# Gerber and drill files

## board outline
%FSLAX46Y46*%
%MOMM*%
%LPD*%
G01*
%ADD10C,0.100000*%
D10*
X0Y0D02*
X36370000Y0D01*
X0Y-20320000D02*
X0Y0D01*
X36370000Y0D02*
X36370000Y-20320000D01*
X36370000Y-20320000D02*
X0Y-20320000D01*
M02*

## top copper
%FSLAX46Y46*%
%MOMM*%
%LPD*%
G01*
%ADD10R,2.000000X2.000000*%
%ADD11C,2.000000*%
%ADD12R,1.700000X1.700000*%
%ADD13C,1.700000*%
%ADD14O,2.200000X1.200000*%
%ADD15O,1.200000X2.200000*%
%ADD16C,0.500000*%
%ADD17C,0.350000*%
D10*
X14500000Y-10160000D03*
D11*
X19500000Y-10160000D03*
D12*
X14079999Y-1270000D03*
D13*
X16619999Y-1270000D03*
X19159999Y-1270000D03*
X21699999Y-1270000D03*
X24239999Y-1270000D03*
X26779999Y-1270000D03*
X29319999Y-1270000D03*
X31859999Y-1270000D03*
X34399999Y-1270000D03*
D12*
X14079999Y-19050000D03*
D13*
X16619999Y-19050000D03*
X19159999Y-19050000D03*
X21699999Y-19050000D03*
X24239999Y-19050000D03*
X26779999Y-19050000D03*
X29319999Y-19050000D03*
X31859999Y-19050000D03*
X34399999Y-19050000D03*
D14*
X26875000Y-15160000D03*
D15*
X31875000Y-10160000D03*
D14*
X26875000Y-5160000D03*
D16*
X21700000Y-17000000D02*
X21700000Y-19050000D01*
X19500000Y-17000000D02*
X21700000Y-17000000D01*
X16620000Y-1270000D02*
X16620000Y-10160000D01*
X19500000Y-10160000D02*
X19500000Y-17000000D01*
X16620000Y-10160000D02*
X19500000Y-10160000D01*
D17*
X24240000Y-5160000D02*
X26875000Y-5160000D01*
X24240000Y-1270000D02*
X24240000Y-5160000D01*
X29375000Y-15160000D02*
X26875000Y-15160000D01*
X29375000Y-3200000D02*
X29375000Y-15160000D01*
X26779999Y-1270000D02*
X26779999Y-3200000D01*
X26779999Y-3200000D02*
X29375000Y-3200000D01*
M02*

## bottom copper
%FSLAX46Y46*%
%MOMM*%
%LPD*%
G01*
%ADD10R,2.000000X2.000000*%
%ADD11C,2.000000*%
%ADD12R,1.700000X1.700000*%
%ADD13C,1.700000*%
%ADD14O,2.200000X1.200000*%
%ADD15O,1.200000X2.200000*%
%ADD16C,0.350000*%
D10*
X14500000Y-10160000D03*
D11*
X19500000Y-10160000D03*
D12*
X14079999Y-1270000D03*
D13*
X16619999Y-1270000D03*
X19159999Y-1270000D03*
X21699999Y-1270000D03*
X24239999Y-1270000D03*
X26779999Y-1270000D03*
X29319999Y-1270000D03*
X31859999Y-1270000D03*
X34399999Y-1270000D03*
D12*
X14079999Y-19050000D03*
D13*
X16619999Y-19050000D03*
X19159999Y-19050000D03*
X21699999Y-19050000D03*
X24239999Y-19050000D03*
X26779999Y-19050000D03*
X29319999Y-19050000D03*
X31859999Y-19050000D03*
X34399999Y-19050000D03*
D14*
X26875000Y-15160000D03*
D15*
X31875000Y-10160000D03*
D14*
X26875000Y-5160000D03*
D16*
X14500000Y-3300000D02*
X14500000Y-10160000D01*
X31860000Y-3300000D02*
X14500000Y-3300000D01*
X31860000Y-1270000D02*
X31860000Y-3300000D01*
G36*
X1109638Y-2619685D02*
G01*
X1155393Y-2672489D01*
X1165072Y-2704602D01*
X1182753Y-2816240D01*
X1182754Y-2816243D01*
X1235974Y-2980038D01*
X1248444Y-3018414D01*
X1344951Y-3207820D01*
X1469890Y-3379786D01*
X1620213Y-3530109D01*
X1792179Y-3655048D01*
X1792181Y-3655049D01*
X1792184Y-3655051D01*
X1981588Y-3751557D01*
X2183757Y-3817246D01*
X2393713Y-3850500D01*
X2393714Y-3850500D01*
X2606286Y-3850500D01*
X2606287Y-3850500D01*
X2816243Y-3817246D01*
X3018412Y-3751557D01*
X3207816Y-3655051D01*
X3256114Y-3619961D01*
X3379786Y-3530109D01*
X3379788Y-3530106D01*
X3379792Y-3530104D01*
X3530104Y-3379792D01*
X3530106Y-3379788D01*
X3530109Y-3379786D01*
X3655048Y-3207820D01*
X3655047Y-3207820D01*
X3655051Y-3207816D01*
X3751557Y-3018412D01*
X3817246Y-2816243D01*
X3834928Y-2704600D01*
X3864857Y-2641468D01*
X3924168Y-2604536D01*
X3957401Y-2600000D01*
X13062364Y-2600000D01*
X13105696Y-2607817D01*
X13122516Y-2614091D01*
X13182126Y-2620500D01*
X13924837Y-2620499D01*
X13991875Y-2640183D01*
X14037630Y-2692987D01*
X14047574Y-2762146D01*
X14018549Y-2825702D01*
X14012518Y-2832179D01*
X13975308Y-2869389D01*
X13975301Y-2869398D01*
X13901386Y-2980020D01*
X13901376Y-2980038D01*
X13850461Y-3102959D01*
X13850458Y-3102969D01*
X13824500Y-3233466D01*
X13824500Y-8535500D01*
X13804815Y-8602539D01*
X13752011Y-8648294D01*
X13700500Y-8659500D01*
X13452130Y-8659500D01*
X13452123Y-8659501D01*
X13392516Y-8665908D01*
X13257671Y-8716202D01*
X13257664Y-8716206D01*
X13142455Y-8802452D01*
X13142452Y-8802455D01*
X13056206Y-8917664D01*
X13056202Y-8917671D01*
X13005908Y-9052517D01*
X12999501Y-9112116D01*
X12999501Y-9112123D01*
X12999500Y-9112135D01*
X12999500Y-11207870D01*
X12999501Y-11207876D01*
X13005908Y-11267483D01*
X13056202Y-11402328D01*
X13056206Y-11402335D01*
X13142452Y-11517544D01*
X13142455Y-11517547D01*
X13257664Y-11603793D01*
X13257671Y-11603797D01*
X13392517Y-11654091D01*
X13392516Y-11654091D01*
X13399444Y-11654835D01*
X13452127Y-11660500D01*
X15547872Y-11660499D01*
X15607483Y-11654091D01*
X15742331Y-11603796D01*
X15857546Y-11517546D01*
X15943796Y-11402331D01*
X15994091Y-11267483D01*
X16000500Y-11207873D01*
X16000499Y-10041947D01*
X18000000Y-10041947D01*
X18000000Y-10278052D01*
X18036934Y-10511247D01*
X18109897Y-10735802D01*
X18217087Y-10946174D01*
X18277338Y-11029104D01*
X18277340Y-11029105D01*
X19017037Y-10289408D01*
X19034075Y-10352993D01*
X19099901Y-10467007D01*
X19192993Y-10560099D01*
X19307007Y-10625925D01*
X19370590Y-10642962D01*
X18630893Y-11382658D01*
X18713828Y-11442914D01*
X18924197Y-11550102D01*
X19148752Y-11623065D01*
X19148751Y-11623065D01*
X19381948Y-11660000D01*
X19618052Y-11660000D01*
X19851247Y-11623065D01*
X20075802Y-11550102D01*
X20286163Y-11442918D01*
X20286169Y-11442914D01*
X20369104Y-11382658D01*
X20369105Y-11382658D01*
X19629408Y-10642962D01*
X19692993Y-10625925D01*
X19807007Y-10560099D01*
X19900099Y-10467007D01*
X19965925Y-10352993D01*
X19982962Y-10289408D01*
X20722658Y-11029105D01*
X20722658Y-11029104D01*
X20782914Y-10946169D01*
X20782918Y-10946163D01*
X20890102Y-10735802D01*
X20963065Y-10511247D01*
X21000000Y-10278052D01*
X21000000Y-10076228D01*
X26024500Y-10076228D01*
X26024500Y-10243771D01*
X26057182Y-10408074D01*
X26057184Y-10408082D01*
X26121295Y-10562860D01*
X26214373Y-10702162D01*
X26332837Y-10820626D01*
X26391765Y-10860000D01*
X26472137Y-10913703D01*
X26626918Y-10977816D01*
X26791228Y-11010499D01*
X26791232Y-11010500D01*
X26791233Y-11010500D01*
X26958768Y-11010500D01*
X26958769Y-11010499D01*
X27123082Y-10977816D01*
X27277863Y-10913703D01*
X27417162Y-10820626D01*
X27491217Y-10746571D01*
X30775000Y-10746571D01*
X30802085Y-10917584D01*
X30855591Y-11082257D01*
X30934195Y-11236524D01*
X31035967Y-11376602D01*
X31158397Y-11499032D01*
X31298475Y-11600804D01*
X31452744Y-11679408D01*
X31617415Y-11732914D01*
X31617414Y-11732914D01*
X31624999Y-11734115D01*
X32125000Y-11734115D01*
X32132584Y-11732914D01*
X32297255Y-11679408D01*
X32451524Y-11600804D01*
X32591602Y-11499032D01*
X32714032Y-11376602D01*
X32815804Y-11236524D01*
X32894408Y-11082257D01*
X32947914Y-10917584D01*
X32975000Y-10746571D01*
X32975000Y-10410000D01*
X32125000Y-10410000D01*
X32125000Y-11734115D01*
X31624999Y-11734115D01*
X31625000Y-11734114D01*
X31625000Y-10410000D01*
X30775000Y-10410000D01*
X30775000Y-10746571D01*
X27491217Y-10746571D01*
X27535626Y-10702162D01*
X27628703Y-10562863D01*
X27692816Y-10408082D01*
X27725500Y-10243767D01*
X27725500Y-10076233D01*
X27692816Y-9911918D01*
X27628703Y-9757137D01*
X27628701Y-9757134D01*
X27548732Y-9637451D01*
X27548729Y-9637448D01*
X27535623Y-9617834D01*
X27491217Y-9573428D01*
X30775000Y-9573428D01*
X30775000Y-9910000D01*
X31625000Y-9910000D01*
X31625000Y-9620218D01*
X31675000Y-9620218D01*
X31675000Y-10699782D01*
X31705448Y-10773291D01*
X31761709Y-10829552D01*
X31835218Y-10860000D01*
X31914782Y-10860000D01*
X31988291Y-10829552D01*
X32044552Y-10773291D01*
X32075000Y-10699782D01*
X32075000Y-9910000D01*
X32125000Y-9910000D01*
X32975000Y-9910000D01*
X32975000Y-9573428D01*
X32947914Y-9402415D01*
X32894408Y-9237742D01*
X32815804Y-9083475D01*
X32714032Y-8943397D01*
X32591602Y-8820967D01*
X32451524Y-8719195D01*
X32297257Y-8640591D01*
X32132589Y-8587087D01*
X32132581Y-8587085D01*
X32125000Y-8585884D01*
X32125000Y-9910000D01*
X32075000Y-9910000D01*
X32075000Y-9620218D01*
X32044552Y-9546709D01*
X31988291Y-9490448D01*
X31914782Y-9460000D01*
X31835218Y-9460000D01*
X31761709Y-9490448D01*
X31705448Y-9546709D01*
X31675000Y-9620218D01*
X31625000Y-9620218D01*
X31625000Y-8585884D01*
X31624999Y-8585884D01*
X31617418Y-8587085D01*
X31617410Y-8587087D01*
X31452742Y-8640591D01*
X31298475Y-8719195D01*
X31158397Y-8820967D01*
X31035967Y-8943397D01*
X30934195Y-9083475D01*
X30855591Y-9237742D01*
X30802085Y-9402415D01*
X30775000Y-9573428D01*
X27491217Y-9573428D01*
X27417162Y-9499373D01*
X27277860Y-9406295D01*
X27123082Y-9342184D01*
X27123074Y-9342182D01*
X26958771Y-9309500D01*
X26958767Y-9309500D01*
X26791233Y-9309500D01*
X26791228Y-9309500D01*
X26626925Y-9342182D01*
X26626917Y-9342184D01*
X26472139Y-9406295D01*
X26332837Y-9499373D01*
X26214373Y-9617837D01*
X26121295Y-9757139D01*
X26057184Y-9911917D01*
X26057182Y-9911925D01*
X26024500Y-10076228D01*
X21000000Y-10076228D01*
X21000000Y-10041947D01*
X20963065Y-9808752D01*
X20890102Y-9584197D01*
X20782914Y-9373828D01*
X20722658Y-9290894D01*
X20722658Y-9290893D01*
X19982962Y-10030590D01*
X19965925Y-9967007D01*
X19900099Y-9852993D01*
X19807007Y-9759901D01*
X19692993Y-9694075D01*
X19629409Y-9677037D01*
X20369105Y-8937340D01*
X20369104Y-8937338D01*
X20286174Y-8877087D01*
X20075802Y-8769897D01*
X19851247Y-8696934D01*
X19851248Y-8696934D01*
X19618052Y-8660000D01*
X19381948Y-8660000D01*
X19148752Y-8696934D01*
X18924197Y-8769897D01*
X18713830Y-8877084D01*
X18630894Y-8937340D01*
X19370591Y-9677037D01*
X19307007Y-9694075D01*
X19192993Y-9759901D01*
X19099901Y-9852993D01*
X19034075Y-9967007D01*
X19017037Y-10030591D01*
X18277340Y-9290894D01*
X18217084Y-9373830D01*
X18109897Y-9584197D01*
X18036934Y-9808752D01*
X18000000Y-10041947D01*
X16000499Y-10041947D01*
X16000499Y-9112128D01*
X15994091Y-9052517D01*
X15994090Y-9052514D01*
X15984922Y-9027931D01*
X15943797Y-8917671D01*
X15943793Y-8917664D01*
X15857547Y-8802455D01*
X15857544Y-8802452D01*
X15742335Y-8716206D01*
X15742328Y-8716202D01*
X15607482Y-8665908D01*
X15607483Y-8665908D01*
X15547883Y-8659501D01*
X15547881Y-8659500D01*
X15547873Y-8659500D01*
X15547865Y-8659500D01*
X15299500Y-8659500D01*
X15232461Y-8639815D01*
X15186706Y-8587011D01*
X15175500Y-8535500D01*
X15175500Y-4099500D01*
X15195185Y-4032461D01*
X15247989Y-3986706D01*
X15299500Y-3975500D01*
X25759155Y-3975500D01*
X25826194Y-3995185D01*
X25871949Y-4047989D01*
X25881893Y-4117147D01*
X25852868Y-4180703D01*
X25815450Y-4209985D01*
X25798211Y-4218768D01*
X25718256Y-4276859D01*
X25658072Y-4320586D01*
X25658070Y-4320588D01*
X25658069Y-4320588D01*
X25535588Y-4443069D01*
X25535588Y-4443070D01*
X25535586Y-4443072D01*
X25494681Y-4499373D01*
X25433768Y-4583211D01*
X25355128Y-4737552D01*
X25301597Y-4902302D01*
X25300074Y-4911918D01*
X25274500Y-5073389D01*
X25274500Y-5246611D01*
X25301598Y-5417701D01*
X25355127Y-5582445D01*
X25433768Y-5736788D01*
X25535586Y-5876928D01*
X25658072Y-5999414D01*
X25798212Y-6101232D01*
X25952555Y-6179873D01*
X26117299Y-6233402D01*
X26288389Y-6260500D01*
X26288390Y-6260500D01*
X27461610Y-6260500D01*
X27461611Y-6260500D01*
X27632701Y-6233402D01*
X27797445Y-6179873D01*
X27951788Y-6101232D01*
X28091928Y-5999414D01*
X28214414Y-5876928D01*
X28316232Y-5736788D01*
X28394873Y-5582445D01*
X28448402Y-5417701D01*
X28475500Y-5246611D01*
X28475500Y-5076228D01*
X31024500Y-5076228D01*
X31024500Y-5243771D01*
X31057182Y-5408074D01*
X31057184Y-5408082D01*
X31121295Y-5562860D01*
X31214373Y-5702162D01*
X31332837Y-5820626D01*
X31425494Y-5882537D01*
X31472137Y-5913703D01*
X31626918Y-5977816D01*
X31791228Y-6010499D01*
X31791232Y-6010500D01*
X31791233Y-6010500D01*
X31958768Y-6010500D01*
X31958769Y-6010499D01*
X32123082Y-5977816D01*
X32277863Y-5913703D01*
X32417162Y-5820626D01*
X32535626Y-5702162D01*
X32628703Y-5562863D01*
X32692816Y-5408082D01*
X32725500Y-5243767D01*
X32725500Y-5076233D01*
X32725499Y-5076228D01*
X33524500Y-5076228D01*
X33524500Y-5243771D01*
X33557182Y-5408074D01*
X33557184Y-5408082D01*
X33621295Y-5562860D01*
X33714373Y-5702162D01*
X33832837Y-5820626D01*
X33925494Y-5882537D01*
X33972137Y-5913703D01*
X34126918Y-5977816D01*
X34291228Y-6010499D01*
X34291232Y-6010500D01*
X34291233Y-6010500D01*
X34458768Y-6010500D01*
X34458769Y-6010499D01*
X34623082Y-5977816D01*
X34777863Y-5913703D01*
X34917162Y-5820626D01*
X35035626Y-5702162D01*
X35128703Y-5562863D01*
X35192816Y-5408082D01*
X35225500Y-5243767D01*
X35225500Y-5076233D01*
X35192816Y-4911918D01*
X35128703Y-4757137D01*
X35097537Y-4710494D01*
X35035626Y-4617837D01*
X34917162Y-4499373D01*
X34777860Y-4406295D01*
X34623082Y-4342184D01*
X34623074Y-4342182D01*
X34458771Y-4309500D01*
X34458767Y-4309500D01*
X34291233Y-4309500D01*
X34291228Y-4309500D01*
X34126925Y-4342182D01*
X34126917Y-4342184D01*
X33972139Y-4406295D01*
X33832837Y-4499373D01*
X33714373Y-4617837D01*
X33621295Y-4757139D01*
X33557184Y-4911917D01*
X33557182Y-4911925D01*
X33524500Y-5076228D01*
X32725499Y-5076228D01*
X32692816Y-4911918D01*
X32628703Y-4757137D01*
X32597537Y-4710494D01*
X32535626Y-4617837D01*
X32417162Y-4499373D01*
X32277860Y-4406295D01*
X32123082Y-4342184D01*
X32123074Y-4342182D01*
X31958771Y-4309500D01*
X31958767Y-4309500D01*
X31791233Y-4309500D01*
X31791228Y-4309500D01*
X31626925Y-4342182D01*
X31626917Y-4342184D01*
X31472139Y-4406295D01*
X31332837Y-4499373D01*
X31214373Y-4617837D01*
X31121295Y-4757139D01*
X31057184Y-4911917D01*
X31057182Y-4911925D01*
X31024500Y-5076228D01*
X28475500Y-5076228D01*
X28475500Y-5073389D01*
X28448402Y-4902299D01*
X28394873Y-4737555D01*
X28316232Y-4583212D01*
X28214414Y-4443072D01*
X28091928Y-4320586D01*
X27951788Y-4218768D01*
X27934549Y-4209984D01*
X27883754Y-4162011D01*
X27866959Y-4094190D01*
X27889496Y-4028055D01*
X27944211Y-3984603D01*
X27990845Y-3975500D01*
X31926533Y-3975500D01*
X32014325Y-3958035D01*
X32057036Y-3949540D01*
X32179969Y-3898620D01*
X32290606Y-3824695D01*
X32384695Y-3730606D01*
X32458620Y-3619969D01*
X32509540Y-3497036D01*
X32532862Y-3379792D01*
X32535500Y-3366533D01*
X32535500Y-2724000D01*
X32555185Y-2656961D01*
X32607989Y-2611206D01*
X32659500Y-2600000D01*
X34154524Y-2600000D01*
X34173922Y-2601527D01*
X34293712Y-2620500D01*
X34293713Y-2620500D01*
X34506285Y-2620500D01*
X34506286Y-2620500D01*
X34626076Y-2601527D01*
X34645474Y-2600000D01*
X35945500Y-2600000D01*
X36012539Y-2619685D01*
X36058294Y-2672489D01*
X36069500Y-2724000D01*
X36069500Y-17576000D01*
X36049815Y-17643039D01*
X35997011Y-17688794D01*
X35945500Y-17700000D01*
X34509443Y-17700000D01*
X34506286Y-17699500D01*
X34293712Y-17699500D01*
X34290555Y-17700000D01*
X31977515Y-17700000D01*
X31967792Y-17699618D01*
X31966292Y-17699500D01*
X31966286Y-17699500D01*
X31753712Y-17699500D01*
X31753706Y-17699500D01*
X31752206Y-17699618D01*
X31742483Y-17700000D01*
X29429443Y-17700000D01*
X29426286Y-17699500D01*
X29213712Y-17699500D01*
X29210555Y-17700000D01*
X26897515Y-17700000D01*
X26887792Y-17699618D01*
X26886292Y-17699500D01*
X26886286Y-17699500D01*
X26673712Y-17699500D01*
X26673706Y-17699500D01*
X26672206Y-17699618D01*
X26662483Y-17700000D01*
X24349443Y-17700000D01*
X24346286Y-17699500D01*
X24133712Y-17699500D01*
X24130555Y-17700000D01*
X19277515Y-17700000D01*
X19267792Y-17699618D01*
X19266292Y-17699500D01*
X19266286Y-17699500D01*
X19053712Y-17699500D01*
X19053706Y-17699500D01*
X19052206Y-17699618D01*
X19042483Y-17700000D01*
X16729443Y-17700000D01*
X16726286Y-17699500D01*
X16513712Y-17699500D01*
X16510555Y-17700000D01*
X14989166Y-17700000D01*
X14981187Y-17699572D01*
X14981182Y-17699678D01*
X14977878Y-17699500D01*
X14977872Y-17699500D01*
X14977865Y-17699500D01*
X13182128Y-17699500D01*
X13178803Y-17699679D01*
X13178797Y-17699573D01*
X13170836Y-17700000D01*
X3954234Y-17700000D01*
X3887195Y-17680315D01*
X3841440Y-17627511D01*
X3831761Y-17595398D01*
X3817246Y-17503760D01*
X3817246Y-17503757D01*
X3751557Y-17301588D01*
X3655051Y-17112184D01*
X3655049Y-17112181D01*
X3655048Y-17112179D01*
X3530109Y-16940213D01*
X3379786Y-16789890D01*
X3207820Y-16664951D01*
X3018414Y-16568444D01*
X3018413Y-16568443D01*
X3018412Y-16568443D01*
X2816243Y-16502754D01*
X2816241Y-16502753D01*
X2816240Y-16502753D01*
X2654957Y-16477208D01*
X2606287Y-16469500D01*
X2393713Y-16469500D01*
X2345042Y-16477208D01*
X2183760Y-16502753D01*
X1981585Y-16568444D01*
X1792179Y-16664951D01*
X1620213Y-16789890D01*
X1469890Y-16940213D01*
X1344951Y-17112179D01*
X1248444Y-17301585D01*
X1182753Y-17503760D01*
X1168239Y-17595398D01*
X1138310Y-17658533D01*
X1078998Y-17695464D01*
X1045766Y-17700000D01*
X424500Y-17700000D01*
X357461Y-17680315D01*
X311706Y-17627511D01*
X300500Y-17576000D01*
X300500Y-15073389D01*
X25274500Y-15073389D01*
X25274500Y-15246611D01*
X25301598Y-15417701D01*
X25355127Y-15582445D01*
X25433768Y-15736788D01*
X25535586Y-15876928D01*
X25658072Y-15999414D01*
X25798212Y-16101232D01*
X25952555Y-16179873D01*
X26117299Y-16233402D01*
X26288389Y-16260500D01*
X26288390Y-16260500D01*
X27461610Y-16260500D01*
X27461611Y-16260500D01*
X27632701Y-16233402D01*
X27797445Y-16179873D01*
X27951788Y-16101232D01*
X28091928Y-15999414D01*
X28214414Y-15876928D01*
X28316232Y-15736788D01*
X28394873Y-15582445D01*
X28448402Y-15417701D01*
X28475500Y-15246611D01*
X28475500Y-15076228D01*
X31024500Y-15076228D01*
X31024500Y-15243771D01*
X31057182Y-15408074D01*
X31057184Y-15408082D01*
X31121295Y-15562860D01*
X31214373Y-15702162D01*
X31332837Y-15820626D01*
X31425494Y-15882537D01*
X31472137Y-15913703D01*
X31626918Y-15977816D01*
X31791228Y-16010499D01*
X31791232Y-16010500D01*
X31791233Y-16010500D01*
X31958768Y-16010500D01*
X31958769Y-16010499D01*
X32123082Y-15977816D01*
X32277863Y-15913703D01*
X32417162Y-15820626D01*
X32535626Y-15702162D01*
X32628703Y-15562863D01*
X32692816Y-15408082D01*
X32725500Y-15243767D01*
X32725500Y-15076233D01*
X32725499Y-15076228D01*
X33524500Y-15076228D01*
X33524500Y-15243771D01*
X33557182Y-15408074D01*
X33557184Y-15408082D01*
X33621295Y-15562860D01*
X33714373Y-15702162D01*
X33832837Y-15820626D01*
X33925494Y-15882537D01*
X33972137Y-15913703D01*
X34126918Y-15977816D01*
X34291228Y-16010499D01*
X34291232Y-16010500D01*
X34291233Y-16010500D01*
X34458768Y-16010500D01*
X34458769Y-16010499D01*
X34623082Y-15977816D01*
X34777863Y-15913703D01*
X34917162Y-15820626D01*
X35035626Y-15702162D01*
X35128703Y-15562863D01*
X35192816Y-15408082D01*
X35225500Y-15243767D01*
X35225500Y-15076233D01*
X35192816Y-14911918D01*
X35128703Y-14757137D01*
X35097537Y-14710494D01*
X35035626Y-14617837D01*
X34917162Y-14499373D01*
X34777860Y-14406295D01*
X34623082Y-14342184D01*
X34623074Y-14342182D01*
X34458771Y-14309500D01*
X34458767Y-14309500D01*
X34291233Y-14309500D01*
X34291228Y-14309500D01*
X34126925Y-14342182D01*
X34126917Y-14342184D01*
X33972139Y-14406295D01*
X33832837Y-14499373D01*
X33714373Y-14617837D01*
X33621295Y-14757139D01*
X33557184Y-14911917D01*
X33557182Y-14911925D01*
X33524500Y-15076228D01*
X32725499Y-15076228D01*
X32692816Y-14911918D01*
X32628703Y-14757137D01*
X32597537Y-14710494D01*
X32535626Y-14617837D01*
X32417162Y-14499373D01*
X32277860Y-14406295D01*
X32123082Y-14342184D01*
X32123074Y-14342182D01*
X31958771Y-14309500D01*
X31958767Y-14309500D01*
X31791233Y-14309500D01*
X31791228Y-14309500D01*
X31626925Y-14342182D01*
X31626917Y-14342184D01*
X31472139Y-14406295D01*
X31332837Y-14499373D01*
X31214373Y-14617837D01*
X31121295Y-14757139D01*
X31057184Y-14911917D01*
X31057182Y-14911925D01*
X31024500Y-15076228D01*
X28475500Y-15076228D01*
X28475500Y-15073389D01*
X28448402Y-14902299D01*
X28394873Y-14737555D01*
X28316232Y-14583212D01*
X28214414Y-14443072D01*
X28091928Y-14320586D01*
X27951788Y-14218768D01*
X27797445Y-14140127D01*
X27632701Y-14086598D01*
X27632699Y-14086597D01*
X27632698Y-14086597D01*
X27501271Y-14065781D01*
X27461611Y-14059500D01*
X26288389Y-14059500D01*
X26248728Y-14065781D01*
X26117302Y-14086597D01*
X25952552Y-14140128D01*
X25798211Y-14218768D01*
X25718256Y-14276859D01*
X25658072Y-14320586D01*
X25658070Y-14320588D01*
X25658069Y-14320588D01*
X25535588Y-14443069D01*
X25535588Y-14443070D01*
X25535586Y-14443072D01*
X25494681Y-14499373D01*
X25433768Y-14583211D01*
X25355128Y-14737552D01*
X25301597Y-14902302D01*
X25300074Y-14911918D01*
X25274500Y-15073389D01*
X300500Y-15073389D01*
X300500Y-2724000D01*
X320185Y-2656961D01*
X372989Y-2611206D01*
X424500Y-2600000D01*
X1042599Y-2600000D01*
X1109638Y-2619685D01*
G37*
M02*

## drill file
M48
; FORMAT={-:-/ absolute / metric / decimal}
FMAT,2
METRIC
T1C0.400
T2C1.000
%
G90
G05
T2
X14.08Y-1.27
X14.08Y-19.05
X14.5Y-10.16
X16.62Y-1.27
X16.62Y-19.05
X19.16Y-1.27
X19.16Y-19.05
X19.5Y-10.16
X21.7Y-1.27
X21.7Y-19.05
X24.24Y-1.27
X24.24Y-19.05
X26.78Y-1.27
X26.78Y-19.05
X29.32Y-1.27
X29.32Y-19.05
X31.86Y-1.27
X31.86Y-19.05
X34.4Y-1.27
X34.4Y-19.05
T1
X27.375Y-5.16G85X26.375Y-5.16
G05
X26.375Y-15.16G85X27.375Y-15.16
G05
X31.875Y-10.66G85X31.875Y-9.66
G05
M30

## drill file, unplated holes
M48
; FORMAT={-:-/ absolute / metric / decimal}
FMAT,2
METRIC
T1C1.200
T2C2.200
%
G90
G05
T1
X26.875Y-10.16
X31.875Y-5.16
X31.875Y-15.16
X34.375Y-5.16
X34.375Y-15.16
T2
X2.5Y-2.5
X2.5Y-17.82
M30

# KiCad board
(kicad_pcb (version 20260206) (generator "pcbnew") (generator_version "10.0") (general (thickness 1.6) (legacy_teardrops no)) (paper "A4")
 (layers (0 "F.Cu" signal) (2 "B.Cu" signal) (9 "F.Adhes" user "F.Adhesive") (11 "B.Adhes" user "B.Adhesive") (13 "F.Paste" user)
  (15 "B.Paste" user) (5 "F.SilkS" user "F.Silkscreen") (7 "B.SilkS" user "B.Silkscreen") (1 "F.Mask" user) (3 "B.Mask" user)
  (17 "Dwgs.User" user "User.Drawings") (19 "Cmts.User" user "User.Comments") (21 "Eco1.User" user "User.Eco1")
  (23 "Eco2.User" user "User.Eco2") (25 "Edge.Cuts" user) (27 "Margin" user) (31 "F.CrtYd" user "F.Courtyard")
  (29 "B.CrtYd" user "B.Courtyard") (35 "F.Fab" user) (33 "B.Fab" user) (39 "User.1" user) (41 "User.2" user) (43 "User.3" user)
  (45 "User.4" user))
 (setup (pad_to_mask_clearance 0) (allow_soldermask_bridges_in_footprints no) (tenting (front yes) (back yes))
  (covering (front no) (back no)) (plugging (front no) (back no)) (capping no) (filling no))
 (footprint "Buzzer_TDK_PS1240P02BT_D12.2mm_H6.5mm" (layer "F.Cu") (at 14.5 10.16)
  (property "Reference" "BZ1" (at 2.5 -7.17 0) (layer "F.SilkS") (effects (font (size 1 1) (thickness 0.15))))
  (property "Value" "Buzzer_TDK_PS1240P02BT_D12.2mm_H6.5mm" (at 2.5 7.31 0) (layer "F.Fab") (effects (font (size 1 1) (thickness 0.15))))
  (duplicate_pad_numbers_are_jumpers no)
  (pad "1" thru_hole rect (at 0 0) (size 2 2) (drill 1) (layers "*.Cu" "*.Mask") (remove_unused_layers no) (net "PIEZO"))
  (pad "2" thru_hole circle (at 5 0) (size 2 2) (drill 1) (layers "*.Cu" "*.Mask") (remove_unused_layers no) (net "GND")))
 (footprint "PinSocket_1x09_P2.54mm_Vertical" (layer "F.Cu") (at 14.079999 1.27 90)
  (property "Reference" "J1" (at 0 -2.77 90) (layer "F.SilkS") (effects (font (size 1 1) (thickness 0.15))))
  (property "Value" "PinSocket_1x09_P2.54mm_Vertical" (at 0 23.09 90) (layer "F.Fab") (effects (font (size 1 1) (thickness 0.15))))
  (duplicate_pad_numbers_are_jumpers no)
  (pad "1" thru_hole rect (at 0 0 90) (size 1.7 1.7) (drill 1) (layers "*.Cu" "*.Mask") (remove_unused_layers no))
  (pad "2" thru_hole circle (at 0 2.54 90) (size 1.7 1.7) (drill 1) (layers "*.Cu" "*.Mask") (remove_unused_layers no) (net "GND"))
  (pad "3" thru_hole circle (at 0 5.08 90) (size 1.7 1.7) (drill 1) (layers "*.Cu" "*.Mask") (remove_unused_layers no))
  (pad "4" thru_hole circle (at 0 7.62 90) (size 1.7 1.7) (drill 1) (layers "*.Cu" "*.Mask") (remove_unused_layers no))
  (pad "5" thru_hole circle (at 0 10.16 90) (size 1.7 1.7) (drill 1) (layers "*.Cu" "*.Mask") (remove_unused_layers no) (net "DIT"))
  (pad "6" thru_hole circle (at 0 12.7 90) (size 1.7 1.7) (drill 1) (layers "*.Cu" "*.Mask") (remove_unused_layers no) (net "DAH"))
  (pad "7" thru_hole circle (at 0 15.24 90) (size 1.7 1.7) (drill 1) (layers "*.Cu" "*.Mask") (remove_unused_layers no) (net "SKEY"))
  (pad "8" thru_hole circle (at 0 17.78 90) (size 1.7 1.7) (drill 1) (layers "*.Cu" "*.Mask") (remove_unused_layers no) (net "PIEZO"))
  (pad "9" thru_hole circle (at 0 20.32 90) (size 1.7 1.7) (drill 1) (layers "*.Cu" "*.Mask") (remove_unused_layers no)))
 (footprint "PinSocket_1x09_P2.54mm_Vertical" (layer "F.Cu") (at 14.079999 19.05 90)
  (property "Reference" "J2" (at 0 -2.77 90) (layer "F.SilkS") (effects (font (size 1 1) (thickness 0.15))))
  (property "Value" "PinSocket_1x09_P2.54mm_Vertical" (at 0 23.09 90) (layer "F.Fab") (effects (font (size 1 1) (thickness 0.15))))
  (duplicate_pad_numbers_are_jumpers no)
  (pad "1" thru_hole rect (at 0 0 90) (size 1.7 1.7) (drill 1) (layers "*.Cu" "*.Mask") (remove_unused_layers no))
  (pad "2" thru_hole circle (at 0 2.54 90) (size 1.7 1.7) (drill 1) (layers "*.Cu" "*.Mask") (remove_unused_layers no))
  (pad "3" thru_hole circle (at 0 5.08 90) (size 1.7 1.7) (drill 1) (layers "*.Cu" "*.Mask") (remove_unused_layers no))
  (pad "4" thru_hole circle (at 0 7.62 90) (size 1.7 1.7) (drill 1) (layers "*.Cu" "*.Mask") (remove_unused_layers no) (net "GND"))
  (pad "5" thru_hole circle (at 0 10.16 90) (size 1.7 1.7) (drill 1) (layers "*.Cu" "*.Mask") (remove_unused_layers no))
  (pad "6" thru_hole circle (at 0 12.7 90) (size 1.7 1.7) (drill 1) (layers "*.Cu" "*.Mask") (remove_unused_layers no))
  (pad "7" thru_hole circle (at 0 15.24 90) (size 1.7 1.7) (drill 1) (layers "*.Cu" "*.Mask") (remove_unused_layers no))
  (pad "8" thru_hole circle (at 0 17.78 90) (size 1.7 1.7) (drill 1) (layers "*.Cu" "*.Mask") (remove_unused_layers no))
  (pad "9" thru_hole circle (at 0 20.32 90) (size 1.7 1.7) (drill 1) (layers "*.Cu" "*.Mask") (remove_unused_layers no)))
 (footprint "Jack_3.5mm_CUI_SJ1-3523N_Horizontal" (layer "F.Cu") (at 31.875 10.16 90)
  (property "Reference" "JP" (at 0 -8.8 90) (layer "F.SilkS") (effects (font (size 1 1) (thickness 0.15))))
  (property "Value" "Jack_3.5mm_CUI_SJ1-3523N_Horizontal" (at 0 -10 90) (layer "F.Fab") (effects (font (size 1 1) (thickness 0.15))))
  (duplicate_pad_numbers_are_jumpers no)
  (pad "" np_thru_hole circle (at -5 0 90) (size 1.2 1.2) (drill 1.2) (layers "*.Cu" "*.Mask"))
  (pad "" np_thru_hole circle (at -5 2.5 90) (size 1.2 1.2) (drill 1.2) (layers "*.Cu" "*.Mask"))
  (pad "" np_thru_hole circle (at 0 -5 90) (size 1.2 1.2) (drill 1.2) (layers "*.Cu" "*.Mask"))
  (pad "" np_thru_hole circle (at 5 0 90) (size 1.2 1.2) (drill 1.2) (layers "*.Cu" "*.Mask"))
  (pad "" np_thru_hole circle (at 5 2.5 90) (size 1.2 1.2) (drill 1.2) (layers "*.Cu" "*.Mask"))
  (pad "R" thru_hole oval (at -5 -5 90) (size 1.2 2.2) (drill oval 0.4 1.4) (layers "*.Cu" "*.Mask") (remove_unused_layers no) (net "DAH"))
  (pad "S" thru_hole oval (at 0 0 90) (size 2.2 1.2) (drill oval 1.4 0.4) (layers "*.Cu" "*.Mask") (remove_unused_layers no) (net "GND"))
  (pad "T" thru_hole oval (at 5 -5 270) (size 1.2 2.2) (drill oval 0.4 1.4) (layers "*.Cu" "*.Mask") (remove_unused_layers no) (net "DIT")))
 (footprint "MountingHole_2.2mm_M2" (layer "F.Cu") (at 2.5 17.82)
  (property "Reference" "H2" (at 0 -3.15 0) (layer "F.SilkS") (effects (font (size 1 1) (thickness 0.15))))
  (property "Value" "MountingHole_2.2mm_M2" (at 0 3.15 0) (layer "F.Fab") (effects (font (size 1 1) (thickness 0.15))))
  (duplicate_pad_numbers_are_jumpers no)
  (pad "" np_thru_hole circle (at 0 0) (size 2.2 2.2) (drill 2.2) (layers "*.Cu" "*.Mask")))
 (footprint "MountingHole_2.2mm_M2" (layer "F.Cu") (at 2.5 2.5)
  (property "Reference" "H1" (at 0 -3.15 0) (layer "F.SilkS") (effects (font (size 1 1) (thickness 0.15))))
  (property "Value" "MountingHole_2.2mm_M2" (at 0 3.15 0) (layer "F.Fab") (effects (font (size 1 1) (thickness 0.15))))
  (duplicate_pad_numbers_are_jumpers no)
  (pad "" np_thru_hole circle (at 0 0) (size 2.2 2.2) (drill 2.2) (layers "*.Cu" "*.Mask")))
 (gr_line (start 0 0) (end 36.37 0) (stroke (width 0.1) (type default)) (layer "Edge.Cuts"))
 (gr_line (start 0 20.32) (end 0 0) (stroke (width 0.1) (type default)) (layer "Edge.Cuts"))
 (gr_line (start 36.37 0) (end 36.37 20.32) (stroke (width 0.1) (type default)) (layer "Edge.Cuts"))
 (gr_line (start 36.37 20.32) (end 0 20.32) (stroke (width 0.1) (type default)) (layer "Edge.Cuts"))
 (segment (start 14.5 3.3) (end 14.5 10.16) (width 0.35) (layer "B.Cu") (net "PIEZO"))
 (segment (start 31.86 3.3) (end 14.5 3.3) (width 0.35) (layer "B.Cu") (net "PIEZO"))
 (segment (start 31.86 1.27) (end 31.86 3.3) (width 0.35) (layer "B.Cu") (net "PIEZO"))
 (segment (start 21.7 17) (end 21.7 19.05) (width 0.5) (layer "F.Cu") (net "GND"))
 (segment (start 19.5 17) (end 21.7 17) (width 0.5) (layer "F.Cu") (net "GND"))
 (segment (start 16.62 1.27) (end 16.62 10.16) (width 0.5) (layer "F.Cu") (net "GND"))
 (segment (start 19.5 10.16) (end 19.5 17) (width 0.5) (layer "F.Cu") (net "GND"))
 (segment (start 16.62 10.16) (end 19.5 10.16) (width 0.5) (layer "F.Cu") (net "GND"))
 (segment (start 24.24 5.16) (end 26.875 5.16) (width 0.35) (layer "F.Cu") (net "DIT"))
 (segment (start 24.24 1.27) (end 24.24 5.16) (width 0.35) (layer "F.Cu") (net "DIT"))
 (segment (start 29.375 15.16) (end 26.875 15.16) (width 0.35) (layer "F.Cu") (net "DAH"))
 (segment (start 29.375 3.2) (end 29.375 15.16) (width 0.35) (layer "F.Cu") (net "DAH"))
 (segment (start 26.779999 1.27) (end 26.779999 3.2) (width 0.35) (layer "F.Cu") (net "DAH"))
 (segment (start 26.779999 3.2) (end 29.375 3.2) (width 0.35) (layer "F.Cu") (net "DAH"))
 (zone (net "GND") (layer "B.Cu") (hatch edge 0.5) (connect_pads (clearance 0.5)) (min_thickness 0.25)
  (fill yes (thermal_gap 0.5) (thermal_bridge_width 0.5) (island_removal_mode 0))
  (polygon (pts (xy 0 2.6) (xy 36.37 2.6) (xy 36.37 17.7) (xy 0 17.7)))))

